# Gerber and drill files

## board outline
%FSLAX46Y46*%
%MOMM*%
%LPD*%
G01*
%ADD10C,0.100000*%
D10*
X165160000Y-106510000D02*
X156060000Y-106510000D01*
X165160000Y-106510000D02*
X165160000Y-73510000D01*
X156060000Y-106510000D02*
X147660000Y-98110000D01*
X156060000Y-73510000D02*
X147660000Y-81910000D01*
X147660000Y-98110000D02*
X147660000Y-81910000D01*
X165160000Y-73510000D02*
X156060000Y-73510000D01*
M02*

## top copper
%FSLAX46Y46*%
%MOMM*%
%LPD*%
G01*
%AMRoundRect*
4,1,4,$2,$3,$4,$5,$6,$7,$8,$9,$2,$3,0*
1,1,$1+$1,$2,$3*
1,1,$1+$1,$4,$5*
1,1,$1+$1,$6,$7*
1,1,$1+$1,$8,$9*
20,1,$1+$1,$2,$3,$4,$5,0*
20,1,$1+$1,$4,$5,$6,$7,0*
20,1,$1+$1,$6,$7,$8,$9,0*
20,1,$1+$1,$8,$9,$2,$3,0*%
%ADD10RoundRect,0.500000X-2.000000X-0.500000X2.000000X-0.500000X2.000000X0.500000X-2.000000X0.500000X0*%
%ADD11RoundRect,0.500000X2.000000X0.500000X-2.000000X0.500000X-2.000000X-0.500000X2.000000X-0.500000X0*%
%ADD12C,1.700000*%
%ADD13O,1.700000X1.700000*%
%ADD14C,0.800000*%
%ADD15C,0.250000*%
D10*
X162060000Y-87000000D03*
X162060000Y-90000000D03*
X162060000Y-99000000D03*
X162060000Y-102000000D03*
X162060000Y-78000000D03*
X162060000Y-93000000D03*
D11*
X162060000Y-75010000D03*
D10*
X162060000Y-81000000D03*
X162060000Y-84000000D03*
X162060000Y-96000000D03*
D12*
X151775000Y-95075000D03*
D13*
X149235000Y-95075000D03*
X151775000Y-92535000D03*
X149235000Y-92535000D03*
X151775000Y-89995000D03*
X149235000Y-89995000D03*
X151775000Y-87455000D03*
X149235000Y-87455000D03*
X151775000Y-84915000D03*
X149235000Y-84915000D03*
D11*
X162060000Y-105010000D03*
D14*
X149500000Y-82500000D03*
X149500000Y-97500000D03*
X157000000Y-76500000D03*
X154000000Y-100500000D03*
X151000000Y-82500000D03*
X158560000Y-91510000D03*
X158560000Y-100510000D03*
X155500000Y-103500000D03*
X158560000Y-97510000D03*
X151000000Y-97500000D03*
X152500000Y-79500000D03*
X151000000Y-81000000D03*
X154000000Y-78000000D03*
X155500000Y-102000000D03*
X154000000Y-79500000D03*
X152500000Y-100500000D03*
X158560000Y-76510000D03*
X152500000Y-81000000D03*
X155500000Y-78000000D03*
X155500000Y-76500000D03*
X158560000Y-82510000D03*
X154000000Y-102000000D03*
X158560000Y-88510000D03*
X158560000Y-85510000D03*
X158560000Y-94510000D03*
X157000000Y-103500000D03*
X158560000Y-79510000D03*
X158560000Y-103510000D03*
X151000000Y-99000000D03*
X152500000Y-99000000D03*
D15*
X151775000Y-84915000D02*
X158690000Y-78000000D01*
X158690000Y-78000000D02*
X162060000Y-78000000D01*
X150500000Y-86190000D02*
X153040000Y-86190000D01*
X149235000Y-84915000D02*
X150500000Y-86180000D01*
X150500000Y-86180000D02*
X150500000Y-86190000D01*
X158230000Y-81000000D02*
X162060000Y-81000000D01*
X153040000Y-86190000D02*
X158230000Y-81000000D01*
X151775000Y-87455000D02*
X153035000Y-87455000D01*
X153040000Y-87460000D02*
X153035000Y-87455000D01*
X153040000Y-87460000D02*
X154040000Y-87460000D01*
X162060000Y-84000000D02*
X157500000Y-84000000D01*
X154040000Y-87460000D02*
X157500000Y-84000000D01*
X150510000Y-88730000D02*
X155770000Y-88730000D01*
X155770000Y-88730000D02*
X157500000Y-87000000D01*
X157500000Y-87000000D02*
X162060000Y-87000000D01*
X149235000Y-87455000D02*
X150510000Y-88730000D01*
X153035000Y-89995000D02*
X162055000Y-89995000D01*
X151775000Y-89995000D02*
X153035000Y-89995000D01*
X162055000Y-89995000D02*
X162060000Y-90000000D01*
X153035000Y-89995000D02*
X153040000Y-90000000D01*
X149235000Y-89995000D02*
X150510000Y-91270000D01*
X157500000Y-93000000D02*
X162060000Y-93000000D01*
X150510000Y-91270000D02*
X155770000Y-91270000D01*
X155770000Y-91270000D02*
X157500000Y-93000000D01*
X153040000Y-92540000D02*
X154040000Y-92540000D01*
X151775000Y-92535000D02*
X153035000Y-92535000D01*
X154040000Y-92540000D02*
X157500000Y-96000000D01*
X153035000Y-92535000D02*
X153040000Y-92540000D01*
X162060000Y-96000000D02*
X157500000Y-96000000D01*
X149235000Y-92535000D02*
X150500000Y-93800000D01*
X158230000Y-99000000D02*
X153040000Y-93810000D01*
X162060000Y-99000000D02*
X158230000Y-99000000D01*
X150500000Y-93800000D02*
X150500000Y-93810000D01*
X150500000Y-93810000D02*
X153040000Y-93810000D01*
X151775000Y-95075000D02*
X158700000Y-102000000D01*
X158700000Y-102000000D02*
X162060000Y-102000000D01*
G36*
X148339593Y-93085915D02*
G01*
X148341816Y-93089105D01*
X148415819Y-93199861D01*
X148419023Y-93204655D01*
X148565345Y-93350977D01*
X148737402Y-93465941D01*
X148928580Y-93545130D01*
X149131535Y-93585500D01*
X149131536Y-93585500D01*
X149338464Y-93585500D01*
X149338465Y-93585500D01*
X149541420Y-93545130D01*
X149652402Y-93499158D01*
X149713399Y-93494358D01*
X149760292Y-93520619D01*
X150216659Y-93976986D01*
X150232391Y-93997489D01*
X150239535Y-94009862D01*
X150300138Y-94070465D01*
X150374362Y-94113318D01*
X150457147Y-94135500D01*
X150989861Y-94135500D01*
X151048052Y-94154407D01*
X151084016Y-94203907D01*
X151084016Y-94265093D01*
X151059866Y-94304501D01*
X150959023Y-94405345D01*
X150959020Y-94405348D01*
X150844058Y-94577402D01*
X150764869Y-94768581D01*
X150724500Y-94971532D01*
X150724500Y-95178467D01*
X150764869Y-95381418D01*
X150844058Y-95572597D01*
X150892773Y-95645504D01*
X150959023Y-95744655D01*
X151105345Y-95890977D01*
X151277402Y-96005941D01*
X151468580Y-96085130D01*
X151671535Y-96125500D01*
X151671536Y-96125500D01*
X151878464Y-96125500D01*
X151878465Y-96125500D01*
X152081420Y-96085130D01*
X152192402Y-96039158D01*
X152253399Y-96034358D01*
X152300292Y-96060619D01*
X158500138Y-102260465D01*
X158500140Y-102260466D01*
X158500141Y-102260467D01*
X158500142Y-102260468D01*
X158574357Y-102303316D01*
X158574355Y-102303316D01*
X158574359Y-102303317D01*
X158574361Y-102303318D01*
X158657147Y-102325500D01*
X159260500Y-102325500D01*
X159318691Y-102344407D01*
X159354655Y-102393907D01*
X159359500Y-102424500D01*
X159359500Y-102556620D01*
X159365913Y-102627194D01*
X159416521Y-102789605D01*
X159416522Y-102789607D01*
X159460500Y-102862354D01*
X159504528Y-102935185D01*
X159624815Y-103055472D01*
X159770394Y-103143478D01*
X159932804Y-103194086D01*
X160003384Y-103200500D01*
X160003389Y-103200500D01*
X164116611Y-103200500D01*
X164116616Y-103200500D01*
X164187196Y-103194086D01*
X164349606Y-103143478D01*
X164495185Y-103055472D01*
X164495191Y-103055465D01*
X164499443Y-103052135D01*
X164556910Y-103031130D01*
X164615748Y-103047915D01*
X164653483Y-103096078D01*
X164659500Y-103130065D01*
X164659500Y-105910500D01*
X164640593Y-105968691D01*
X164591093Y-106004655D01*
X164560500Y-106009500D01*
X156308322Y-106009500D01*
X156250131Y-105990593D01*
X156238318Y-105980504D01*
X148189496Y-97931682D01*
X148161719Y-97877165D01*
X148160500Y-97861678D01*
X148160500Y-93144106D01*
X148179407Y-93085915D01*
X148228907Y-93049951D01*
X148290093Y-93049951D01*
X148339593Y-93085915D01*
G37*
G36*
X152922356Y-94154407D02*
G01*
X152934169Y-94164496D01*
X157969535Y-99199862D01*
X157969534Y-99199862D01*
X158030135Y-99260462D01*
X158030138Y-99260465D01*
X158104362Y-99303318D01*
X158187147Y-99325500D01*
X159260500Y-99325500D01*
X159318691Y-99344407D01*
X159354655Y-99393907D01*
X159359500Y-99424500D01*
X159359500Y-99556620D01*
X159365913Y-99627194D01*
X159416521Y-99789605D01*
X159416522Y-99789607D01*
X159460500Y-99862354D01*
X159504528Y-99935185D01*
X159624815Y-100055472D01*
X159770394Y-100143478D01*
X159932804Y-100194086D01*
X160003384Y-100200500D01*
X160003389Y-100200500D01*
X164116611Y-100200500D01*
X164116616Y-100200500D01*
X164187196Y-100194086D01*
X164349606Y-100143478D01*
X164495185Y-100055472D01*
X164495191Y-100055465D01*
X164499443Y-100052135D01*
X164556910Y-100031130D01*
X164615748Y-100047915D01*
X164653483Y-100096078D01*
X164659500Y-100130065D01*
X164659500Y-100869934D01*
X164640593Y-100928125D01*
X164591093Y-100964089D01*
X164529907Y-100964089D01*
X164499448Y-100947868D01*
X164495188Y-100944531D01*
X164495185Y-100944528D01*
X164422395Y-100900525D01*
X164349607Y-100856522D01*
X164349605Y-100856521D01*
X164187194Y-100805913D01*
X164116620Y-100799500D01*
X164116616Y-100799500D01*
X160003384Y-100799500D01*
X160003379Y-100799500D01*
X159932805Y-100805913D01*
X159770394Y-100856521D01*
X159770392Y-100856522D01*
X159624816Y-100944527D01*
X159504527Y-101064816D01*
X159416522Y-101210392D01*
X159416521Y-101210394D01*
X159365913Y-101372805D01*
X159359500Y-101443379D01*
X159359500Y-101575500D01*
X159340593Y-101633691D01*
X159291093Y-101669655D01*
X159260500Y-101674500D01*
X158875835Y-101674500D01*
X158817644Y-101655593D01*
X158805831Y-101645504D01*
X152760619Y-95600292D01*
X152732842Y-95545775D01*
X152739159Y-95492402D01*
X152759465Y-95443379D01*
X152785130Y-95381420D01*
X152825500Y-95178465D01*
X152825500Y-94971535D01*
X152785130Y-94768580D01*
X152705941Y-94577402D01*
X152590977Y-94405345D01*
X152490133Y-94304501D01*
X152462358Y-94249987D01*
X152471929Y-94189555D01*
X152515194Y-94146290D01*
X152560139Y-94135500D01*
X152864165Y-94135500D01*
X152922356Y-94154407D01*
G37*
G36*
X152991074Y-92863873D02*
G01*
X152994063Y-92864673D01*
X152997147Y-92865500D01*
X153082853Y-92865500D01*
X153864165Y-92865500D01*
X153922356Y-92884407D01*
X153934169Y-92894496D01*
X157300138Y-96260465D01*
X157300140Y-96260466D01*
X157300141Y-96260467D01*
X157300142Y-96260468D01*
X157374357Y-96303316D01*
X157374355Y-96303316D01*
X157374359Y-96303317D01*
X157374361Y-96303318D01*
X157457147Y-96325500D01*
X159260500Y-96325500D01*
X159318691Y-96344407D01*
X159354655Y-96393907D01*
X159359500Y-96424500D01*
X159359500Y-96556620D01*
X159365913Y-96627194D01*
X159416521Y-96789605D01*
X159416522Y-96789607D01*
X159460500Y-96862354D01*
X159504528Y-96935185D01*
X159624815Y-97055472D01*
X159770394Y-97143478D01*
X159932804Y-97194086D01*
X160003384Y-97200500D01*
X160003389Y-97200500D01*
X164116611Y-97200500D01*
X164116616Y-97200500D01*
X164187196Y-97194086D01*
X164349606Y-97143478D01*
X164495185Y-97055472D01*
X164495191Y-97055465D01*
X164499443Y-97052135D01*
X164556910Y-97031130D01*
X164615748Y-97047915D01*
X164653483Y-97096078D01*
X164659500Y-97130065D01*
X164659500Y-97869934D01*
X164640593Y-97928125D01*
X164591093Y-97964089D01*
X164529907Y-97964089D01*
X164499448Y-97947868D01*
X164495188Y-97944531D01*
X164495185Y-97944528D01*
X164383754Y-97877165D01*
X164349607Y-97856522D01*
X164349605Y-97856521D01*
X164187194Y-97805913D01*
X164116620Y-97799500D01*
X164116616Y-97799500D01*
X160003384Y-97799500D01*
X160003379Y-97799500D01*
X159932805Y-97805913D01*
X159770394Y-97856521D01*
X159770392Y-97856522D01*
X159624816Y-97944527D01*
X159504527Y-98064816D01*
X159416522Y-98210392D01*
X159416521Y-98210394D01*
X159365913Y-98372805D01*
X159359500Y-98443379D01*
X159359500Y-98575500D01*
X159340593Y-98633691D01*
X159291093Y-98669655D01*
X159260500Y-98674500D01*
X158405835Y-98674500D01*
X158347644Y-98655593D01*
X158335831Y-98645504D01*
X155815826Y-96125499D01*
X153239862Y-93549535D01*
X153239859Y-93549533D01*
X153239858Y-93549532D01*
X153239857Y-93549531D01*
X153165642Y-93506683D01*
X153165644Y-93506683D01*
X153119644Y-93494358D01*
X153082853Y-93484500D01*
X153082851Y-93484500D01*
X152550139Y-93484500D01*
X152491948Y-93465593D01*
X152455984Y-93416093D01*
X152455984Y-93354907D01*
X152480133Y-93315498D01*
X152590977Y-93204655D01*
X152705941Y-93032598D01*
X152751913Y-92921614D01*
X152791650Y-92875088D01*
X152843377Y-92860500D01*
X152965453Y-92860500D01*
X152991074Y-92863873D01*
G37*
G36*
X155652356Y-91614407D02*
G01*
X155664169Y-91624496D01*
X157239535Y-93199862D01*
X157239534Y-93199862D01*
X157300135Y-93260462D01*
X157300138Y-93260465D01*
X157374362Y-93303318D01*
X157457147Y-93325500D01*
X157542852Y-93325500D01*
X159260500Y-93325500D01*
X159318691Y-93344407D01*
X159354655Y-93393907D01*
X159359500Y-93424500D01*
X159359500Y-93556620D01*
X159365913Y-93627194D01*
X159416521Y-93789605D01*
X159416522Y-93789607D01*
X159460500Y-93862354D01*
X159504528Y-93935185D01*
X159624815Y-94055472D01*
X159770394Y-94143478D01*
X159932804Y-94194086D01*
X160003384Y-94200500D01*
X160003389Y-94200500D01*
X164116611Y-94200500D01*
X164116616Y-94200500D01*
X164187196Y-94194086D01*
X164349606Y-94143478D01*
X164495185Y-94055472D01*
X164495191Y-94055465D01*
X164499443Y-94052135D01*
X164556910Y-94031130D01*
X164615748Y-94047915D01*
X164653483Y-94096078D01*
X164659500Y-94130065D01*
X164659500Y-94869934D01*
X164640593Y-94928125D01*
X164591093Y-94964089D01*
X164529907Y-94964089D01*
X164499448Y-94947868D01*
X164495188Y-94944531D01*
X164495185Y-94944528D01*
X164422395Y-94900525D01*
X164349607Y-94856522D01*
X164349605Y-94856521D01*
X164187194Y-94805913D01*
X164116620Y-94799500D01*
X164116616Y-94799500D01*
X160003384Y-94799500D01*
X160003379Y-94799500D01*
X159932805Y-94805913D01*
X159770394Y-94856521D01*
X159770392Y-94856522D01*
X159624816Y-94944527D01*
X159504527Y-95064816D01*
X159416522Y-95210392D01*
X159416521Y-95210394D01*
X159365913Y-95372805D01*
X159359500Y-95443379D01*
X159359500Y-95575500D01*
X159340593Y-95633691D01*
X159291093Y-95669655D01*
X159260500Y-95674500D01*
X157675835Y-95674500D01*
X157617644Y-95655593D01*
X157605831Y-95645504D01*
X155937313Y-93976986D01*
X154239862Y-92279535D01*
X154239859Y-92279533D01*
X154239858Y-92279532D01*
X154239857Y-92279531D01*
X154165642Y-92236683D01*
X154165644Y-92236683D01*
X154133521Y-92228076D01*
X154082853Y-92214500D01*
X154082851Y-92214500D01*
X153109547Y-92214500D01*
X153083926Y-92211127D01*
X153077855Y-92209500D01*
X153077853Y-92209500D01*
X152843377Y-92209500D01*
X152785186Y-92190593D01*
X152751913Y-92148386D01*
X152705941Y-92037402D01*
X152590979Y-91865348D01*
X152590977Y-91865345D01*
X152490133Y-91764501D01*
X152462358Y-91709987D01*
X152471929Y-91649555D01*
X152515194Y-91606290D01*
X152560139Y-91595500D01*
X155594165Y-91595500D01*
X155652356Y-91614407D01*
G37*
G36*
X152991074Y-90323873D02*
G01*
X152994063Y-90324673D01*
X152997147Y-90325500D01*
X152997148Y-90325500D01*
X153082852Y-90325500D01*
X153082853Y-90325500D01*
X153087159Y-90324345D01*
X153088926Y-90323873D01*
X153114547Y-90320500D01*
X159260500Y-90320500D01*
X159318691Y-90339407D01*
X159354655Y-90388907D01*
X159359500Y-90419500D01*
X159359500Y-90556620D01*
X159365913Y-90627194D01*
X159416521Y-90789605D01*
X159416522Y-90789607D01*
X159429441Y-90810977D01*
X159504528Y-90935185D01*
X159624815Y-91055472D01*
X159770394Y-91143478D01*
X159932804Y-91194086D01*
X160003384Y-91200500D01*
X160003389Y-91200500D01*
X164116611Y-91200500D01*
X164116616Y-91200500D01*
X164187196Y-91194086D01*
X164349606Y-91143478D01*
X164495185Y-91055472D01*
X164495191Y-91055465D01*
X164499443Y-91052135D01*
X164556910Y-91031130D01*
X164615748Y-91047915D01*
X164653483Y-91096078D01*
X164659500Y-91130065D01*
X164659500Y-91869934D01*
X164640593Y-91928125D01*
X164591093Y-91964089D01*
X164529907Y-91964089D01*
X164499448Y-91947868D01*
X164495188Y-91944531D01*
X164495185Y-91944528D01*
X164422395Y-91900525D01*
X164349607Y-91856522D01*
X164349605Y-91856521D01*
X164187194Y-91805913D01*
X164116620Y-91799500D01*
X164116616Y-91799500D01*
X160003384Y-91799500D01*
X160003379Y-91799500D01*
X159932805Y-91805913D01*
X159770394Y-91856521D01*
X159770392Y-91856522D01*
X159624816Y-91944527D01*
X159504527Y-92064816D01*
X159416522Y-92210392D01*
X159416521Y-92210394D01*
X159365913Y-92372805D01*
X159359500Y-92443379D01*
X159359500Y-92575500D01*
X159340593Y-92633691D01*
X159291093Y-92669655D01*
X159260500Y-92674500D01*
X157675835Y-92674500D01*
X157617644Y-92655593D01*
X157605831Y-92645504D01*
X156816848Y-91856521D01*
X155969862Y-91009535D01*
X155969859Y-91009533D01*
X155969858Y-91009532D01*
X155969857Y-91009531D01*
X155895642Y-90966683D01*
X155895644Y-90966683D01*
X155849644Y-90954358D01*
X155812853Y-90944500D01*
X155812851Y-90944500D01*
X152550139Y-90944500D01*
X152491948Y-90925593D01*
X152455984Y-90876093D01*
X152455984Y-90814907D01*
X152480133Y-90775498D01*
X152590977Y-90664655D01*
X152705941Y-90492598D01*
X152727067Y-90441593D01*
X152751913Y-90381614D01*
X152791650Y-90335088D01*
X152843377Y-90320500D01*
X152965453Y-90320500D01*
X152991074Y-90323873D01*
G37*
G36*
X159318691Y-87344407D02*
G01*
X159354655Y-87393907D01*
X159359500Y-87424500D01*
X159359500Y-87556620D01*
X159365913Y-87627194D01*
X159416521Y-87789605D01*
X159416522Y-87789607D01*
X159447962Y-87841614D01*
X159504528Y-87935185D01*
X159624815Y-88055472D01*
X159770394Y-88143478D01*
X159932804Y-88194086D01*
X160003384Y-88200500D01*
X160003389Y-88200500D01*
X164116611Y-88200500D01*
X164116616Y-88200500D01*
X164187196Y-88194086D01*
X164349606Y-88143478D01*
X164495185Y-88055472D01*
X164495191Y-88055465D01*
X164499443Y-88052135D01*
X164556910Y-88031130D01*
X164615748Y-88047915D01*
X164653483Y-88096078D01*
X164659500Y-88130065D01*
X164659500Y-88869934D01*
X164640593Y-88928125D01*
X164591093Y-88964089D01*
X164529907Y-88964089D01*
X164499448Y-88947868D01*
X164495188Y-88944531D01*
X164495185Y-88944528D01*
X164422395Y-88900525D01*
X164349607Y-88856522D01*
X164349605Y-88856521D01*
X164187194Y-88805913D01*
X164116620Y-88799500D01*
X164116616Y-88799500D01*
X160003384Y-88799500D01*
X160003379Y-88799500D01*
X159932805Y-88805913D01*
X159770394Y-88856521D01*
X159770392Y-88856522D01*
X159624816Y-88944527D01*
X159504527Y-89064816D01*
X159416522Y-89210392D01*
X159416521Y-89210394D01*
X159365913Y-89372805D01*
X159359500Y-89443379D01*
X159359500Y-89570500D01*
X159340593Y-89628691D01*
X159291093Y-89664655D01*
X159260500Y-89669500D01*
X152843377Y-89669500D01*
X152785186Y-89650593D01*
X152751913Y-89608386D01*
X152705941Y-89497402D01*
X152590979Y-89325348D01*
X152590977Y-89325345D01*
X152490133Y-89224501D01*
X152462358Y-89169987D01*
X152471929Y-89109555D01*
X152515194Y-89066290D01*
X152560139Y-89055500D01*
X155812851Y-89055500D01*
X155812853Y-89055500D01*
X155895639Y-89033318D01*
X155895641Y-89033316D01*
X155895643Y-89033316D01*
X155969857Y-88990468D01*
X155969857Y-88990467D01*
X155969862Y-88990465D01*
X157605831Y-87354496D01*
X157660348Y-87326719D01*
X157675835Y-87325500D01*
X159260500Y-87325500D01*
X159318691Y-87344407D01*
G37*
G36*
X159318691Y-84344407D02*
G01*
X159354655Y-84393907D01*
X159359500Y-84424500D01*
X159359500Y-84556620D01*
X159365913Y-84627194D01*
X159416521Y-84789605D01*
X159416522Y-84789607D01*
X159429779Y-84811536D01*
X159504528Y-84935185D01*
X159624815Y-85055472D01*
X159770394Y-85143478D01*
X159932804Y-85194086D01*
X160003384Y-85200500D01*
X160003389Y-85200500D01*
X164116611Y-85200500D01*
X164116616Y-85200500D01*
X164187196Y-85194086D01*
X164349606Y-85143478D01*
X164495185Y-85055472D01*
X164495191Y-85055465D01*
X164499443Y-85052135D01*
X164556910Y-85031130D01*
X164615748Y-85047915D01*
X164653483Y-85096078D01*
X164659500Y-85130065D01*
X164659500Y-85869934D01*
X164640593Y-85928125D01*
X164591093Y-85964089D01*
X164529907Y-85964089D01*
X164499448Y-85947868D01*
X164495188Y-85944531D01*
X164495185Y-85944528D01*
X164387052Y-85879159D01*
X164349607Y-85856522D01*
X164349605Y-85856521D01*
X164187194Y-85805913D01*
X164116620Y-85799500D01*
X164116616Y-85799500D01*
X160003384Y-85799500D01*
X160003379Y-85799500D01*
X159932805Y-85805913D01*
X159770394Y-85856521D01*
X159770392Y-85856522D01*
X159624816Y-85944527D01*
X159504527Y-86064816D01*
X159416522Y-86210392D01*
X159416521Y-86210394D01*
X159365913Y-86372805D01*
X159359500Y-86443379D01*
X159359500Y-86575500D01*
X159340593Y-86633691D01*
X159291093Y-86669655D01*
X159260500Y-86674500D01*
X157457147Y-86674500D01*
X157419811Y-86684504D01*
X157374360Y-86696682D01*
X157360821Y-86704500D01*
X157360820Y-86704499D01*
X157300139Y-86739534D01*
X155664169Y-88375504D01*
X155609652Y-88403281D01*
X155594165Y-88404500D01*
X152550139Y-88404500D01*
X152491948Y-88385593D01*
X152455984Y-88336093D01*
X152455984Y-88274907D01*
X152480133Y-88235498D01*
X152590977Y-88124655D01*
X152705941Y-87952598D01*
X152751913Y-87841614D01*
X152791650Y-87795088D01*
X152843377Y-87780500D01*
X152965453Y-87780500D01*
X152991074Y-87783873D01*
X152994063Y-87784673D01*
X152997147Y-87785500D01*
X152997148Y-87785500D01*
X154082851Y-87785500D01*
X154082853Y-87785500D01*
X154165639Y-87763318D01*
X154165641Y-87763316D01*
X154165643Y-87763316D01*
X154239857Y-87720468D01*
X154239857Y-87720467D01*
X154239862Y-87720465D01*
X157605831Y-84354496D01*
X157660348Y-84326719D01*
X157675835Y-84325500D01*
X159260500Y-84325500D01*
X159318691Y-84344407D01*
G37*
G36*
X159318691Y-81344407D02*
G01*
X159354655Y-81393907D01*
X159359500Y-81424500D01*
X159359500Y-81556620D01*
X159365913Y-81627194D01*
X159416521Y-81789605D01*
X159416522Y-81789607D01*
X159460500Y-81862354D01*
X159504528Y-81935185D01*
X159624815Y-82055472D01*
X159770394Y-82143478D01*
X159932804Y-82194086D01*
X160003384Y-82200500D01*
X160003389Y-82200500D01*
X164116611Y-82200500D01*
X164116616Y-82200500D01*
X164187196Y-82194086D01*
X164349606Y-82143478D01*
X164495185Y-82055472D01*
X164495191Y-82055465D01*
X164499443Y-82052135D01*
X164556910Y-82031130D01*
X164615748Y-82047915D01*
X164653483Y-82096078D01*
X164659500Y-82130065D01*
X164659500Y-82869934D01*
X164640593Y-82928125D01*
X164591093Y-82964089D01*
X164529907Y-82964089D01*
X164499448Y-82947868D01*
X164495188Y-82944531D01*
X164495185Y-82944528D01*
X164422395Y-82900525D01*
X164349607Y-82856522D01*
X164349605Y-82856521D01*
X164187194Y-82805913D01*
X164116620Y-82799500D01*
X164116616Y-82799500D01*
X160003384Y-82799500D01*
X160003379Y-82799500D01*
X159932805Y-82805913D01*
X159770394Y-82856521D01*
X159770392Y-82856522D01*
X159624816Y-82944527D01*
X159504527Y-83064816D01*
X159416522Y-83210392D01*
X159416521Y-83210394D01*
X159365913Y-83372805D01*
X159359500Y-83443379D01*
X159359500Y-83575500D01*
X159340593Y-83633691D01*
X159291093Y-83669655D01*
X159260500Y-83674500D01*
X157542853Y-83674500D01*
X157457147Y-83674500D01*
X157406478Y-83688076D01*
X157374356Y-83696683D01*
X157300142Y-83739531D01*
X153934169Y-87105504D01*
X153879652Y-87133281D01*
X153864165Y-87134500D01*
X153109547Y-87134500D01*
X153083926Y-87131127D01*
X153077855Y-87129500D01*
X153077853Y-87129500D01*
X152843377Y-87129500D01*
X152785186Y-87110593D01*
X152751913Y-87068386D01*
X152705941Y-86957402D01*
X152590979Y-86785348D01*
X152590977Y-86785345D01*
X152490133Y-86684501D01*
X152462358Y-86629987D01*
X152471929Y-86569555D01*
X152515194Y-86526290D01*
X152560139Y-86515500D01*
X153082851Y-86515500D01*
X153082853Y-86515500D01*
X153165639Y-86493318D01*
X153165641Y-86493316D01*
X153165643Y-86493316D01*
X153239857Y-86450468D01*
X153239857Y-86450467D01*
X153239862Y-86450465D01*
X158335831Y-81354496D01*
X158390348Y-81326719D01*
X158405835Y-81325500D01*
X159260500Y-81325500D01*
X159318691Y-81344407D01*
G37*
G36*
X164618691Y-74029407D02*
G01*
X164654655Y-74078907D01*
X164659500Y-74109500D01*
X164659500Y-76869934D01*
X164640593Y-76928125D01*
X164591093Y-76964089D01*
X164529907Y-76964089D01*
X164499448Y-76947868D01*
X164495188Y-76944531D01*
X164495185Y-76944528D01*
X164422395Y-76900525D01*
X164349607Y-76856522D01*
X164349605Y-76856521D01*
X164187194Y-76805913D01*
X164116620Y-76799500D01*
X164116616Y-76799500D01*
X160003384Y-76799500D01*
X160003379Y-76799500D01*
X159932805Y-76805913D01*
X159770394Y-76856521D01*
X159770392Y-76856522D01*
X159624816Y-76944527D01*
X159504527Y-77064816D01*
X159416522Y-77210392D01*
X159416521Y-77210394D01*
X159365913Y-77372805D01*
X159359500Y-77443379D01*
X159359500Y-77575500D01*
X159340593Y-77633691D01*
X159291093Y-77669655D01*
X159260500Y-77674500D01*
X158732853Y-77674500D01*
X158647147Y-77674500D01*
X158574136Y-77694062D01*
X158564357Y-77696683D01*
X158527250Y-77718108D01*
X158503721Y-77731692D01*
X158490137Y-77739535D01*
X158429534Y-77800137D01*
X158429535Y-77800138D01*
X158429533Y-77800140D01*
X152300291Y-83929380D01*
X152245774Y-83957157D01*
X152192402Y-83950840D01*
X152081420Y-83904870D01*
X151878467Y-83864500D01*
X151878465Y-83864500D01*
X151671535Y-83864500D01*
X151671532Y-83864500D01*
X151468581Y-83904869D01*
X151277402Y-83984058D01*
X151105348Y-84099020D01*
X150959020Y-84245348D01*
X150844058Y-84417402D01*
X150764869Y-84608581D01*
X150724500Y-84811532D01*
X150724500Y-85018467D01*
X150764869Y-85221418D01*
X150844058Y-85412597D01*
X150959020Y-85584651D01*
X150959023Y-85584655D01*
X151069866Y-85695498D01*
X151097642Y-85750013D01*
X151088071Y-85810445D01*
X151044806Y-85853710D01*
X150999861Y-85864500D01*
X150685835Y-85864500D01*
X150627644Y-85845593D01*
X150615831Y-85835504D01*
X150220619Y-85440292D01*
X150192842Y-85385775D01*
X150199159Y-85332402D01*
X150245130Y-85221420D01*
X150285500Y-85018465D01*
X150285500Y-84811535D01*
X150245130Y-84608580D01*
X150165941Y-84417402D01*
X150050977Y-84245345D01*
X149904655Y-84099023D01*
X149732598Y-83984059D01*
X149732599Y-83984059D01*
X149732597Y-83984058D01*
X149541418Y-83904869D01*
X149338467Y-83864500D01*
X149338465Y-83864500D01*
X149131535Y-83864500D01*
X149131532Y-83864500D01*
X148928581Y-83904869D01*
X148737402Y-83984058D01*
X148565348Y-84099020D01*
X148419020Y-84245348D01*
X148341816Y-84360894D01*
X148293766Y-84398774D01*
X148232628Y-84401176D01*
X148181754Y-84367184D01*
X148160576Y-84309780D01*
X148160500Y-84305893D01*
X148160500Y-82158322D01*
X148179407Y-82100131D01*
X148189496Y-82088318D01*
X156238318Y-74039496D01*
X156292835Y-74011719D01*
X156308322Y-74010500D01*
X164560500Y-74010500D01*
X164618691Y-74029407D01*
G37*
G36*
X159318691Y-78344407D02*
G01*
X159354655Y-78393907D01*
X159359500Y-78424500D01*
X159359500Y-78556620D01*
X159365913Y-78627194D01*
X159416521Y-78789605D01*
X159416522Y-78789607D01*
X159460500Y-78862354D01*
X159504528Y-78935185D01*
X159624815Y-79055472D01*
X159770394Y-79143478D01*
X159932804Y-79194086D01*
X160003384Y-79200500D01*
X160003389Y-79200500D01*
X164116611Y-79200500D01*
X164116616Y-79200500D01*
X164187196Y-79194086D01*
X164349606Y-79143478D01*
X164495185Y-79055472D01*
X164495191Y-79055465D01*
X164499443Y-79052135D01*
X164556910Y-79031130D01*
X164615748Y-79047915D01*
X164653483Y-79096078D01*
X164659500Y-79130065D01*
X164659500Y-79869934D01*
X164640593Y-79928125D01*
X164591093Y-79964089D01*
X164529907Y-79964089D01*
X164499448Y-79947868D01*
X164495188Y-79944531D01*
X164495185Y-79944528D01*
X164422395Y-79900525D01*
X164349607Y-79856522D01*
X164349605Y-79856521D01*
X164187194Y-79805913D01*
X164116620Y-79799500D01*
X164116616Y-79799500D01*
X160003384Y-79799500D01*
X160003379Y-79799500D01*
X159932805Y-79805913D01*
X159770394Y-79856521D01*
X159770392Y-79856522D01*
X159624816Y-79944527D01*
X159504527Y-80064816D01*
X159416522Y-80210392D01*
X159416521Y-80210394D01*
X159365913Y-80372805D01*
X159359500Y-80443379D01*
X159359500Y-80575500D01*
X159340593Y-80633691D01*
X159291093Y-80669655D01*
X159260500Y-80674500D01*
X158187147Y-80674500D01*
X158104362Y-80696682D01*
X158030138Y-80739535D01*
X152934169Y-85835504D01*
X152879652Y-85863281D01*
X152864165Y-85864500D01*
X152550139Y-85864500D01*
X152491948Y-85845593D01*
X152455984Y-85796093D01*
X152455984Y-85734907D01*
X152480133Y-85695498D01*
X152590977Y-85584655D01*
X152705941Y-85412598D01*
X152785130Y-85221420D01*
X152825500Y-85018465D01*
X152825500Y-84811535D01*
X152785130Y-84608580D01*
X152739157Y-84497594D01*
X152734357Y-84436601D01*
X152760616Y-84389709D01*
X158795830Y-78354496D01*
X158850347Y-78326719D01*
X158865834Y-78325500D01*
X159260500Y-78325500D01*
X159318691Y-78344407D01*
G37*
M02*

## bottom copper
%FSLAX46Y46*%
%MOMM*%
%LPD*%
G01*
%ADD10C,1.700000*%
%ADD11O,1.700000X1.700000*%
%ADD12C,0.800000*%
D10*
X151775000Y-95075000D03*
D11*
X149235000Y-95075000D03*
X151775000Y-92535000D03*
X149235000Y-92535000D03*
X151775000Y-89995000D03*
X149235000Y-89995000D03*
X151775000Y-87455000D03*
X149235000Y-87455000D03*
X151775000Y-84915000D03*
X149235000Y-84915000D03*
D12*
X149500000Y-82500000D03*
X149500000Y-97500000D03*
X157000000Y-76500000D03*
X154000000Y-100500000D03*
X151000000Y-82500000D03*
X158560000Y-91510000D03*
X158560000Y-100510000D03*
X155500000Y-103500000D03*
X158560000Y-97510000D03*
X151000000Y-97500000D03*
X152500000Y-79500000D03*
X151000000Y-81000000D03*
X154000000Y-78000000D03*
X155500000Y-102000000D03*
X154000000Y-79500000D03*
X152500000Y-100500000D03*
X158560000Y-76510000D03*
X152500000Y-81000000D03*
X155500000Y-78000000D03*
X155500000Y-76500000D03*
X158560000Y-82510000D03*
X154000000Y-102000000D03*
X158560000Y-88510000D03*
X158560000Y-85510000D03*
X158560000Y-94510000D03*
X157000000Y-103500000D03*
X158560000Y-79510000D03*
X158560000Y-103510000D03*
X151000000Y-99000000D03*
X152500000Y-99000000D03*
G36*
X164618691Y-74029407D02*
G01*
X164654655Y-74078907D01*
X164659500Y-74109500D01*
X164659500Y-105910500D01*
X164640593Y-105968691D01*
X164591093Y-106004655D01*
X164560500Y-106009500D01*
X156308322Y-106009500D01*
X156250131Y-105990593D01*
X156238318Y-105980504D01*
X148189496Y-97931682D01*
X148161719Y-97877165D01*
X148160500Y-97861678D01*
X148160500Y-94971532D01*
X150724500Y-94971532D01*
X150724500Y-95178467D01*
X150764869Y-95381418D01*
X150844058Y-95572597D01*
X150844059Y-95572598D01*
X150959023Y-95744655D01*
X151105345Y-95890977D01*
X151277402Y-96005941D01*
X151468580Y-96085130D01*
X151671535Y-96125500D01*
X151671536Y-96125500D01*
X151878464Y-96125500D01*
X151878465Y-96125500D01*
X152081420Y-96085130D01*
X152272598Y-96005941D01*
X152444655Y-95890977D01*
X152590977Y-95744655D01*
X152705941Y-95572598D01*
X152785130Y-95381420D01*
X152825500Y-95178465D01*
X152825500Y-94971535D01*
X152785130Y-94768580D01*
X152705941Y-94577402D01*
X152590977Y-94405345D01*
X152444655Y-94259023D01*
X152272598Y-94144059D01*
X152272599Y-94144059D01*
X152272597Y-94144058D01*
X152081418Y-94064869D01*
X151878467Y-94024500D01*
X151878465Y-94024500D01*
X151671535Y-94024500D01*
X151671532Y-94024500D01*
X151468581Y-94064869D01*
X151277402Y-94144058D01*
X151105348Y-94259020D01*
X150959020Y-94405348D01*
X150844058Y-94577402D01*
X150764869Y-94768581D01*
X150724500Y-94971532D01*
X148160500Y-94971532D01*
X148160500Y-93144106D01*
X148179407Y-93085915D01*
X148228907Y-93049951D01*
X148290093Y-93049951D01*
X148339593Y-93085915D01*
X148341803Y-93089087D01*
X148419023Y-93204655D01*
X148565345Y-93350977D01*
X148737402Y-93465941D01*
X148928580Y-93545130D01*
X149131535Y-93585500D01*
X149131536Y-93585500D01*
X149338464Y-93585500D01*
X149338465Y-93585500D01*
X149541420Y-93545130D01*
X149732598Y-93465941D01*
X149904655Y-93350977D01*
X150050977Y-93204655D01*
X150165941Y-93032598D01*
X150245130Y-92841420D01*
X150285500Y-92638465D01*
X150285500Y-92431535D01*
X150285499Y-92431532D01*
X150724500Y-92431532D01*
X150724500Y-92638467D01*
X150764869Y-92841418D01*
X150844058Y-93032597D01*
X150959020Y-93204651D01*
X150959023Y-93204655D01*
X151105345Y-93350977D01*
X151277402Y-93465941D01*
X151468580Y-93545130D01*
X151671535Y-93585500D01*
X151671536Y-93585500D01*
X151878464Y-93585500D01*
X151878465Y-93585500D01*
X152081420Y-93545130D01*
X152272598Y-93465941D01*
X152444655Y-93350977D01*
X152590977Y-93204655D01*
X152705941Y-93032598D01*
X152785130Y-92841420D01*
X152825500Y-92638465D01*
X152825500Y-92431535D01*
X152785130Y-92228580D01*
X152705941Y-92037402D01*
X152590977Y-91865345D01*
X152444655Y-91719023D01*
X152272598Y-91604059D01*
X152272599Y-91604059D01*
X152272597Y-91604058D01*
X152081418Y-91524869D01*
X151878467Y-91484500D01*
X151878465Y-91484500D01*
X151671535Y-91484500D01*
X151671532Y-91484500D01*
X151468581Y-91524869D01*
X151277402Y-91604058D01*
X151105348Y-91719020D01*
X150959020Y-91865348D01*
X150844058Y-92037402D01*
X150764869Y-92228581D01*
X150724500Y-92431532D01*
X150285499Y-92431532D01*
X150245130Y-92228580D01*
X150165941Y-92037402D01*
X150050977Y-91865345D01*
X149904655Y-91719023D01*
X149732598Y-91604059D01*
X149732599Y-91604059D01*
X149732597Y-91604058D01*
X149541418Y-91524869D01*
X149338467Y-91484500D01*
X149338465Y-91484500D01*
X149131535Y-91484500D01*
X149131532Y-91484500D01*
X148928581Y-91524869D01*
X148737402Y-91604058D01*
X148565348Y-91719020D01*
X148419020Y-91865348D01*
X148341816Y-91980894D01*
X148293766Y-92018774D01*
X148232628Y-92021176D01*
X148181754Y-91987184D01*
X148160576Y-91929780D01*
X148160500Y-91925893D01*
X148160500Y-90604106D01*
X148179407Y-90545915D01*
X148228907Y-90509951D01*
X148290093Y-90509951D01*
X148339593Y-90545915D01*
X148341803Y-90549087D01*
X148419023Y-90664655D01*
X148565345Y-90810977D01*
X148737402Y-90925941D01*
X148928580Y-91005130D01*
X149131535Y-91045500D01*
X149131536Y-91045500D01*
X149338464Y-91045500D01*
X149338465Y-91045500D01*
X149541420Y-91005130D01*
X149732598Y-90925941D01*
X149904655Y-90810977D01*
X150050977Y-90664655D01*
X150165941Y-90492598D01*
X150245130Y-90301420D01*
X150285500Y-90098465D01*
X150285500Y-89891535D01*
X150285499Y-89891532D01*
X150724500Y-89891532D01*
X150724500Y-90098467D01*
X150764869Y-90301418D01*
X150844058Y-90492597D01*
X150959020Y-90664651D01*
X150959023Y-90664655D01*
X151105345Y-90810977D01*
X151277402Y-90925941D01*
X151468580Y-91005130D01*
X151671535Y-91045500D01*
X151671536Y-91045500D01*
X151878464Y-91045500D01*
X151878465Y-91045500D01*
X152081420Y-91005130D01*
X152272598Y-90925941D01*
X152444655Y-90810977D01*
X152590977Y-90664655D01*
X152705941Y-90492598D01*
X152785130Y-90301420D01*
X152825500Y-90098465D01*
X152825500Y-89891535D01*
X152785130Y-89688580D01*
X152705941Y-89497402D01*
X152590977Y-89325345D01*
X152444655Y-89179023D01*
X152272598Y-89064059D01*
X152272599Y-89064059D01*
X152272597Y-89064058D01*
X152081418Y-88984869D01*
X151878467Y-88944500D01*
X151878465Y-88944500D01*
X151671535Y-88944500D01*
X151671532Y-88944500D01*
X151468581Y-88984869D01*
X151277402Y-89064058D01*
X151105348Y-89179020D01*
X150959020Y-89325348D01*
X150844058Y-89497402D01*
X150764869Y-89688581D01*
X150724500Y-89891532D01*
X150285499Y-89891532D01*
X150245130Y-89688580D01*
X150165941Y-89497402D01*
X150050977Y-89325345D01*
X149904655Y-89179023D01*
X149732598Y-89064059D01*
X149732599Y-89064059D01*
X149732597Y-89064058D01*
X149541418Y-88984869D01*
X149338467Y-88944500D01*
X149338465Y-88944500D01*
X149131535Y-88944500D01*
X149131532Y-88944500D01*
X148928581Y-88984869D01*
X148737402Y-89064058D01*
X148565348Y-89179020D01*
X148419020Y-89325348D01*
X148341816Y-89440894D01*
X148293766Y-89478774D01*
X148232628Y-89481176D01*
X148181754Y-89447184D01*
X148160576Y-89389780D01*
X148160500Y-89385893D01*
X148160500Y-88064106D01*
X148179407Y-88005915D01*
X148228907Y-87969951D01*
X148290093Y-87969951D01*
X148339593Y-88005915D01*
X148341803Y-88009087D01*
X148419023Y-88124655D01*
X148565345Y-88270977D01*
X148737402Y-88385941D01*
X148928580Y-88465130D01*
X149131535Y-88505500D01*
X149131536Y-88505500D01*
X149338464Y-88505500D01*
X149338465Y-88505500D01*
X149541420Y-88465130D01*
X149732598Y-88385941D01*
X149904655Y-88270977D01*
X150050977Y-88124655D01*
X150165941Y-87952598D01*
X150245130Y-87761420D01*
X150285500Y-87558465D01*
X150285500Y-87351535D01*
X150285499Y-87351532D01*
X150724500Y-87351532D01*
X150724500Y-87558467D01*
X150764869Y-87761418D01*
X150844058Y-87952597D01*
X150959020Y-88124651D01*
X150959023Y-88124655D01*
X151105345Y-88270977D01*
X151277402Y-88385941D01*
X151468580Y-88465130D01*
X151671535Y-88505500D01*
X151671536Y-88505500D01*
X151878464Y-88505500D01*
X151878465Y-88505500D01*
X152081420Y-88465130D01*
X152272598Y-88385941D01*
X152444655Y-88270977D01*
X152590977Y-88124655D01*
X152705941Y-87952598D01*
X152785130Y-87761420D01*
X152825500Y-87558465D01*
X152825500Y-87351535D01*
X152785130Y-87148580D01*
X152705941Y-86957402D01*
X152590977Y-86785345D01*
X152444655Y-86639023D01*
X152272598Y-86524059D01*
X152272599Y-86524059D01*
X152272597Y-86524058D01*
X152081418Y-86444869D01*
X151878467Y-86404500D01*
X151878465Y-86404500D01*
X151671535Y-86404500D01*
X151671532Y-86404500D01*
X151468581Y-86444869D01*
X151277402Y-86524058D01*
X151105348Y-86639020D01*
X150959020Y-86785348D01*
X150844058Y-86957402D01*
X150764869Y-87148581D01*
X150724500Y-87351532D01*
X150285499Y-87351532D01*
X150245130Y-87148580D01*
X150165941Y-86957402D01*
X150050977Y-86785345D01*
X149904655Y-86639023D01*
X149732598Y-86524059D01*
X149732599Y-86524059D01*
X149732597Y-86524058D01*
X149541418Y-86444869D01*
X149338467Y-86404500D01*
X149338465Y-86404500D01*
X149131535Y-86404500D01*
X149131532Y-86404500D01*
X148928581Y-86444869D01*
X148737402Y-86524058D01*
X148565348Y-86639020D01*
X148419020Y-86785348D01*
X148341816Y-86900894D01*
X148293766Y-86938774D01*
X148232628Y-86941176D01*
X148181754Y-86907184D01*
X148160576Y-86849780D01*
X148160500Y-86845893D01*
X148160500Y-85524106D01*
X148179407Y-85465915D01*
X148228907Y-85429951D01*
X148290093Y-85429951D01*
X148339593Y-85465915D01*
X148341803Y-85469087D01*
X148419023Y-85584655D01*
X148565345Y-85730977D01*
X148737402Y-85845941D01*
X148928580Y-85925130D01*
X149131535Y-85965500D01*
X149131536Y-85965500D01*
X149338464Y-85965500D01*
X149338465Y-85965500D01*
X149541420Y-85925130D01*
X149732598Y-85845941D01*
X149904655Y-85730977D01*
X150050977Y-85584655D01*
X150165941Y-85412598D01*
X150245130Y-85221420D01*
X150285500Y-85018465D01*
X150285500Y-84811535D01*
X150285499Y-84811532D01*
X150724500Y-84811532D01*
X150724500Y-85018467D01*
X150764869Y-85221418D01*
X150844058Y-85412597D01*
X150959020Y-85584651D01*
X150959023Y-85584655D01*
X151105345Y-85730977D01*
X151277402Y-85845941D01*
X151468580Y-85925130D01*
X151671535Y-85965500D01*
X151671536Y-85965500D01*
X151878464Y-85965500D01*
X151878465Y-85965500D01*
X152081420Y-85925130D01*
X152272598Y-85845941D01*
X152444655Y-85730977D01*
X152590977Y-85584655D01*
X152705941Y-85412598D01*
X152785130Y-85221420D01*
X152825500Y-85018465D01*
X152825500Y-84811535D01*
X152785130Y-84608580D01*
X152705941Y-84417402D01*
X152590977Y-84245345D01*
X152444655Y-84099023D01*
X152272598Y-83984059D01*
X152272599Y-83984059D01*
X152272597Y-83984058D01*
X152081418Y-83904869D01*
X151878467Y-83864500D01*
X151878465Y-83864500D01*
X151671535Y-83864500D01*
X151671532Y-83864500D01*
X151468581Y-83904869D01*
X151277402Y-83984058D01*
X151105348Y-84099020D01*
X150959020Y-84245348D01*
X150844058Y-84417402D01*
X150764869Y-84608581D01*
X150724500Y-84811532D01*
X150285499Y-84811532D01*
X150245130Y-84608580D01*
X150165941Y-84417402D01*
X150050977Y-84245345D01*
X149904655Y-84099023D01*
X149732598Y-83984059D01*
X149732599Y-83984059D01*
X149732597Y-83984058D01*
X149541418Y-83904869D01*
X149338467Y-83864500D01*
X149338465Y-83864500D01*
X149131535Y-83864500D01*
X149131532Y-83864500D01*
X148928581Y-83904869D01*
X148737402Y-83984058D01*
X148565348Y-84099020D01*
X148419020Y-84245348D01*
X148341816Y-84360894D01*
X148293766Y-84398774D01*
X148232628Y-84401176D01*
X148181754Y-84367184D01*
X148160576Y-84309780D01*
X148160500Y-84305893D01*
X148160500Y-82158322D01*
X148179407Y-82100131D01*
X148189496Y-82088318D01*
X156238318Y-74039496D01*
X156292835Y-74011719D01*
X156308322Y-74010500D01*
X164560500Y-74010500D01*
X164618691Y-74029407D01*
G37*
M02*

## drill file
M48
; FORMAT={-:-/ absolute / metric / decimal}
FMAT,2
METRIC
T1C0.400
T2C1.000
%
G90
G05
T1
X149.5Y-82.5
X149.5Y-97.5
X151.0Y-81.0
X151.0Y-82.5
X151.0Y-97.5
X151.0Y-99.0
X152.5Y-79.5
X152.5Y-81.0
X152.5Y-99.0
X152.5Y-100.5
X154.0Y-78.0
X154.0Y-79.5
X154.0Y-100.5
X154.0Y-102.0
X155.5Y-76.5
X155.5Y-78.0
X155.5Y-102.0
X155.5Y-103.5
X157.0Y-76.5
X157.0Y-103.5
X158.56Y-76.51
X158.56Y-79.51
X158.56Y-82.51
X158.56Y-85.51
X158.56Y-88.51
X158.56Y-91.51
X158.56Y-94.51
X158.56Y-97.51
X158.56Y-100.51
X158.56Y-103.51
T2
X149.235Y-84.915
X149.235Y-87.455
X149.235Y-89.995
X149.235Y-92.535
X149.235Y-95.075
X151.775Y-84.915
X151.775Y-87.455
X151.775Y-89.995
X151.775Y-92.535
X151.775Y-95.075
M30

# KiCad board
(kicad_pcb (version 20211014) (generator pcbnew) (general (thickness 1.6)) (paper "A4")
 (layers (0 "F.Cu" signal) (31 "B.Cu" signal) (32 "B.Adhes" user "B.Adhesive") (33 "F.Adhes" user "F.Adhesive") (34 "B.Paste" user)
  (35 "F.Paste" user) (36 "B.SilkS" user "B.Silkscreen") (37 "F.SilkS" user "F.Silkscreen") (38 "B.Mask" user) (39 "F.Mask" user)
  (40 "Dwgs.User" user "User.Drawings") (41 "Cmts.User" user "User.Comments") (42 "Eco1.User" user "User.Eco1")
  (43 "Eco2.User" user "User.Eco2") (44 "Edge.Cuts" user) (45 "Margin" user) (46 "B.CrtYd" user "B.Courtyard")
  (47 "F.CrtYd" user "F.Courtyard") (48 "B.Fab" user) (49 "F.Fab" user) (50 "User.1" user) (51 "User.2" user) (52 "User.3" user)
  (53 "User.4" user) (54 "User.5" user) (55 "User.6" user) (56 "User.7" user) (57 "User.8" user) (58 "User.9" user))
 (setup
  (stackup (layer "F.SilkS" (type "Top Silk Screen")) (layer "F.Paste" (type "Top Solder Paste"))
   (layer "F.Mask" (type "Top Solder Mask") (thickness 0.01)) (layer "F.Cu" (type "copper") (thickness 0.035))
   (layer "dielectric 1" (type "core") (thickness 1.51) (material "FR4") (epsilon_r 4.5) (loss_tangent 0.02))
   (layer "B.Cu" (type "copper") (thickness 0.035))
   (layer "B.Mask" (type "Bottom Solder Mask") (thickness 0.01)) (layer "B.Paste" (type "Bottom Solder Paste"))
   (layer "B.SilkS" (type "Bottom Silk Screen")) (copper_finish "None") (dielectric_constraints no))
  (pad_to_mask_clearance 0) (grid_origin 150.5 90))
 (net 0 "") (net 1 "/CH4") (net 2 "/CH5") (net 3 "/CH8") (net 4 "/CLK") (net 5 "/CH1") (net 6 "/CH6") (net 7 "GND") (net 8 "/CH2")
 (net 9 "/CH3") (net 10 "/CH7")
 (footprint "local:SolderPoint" (layer "F.Cu") (at 162.06 87)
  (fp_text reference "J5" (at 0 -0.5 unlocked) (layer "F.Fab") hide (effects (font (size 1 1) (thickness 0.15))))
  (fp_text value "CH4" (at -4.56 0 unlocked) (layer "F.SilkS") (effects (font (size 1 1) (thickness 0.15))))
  (pad "1" smd roundrect (at 0 0) (size 5 2) (layers "F.Cu" "F.Paste" "F.Mask") (roundrect_rratio 0.25) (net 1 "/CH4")))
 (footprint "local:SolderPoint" (layer "F.Cu") (at 162.06 90)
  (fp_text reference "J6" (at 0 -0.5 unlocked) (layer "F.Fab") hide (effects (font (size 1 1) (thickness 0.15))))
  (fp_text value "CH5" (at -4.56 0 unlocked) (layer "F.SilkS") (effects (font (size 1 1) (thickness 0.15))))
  (pad "1" smd roundrect (at 0 0) (size 5 2) (layers "F.Cu" "F.Paste" "F.Mask") (roundrect_rratio 0.25) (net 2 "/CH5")))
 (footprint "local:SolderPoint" (layer "F.Cu") (at 162.06 99)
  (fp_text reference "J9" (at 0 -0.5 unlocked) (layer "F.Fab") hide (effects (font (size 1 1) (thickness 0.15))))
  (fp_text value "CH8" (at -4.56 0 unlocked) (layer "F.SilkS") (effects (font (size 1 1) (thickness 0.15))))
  (pad "1" smd roundrect (at 0 0) (size 5 2) (layers "F.Cu" "F.Paste" "F.Mask") (roundrect_rratio 0.25) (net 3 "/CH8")))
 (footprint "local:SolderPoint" (layer "F.Cu") (at 162.06 102)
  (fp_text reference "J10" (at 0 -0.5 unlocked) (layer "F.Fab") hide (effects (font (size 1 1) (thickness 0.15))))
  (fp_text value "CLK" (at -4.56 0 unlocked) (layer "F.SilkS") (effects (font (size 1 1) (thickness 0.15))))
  (pad "1" smd roundrect (at 0 0) (size 5 2) (layers "F.Cu" "F.Paste" "F.Mask") (roundrect_rratio 0.25) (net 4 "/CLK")))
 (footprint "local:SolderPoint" (layer "F.Cu") (at 162.06 78)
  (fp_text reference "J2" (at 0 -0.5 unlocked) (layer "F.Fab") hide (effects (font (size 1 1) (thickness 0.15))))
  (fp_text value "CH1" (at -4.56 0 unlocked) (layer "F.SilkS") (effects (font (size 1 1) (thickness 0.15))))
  (pad "1" smd roundrect (at 0 0) (size 5 2) (layers "F.Cu" "F.Paste" "F.Mask") (roundrect_rratio 0.25) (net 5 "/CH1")))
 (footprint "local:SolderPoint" (layer "F.Cu") (at 162.06 93)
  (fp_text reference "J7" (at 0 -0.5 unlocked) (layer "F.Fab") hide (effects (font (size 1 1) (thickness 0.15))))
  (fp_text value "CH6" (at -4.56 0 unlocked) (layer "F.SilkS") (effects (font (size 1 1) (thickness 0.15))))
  (pad "1" smd roundrect (at 0 0) (size 5 2) (layers "F.Cu" "F.Paste" "F.Mask") (roundrect_rratio 0.25) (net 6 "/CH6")))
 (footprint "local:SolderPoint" (layer "F.Cu") (at 162.06 75.01 180)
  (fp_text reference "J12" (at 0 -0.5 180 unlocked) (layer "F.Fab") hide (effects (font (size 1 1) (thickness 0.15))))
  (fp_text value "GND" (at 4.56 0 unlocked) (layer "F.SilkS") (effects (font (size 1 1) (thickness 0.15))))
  (pad "1" smd roundrect (at 0 0 180) (size 5 2) (layers "F.Cu" "F.Paste" "F.Mask") (roundrect_rratio 0.25) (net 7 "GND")))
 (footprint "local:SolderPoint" (layer "F.Cu") (at 162.06 81)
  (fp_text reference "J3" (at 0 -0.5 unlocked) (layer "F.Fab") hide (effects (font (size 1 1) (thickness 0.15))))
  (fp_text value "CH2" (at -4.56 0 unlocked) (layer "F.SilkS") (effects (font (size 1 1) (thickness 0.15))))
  (pad "1" smd roundrect (at 0 0) (size 5 2) (layers "F.Cu" "F.Paste" "F.Mask") (roundrect_rratio 0.25) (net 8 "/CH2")))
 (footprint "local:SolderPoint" (layer "F.Cu") (at 162.06 84)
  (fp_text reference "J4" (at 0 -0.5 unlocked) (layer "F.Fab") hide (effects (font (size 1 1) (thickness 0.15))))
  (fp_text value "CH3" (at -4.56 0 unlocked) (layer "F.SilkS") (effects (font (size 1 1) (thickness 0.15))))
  (pad "1" smd roundrect (at 0 0) (size 5 2) (layers "F.Cu" "F.Paste" "F.Mask") (roundrect_rratio 0.25) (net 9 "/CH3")))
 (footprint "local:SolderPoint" (layer "F.Cu") (at 162.06 96)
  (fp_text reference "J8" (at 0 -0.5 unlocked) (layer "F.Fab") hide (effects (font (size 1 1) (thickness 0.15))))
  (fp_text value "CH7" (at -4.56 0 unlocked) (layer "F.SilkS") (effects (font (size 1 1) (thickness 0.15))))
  (pad "1" smd roundrect (at 0 0) (size 5 2) (layers "F.Cu" "F.Paste" "F.Mask") (roundrect_rratio 0.25) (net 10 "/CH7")))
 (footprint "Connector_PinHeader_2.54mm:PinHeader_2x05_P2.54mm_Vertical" (layer "F.Cu") (at 151.775 95.075 180)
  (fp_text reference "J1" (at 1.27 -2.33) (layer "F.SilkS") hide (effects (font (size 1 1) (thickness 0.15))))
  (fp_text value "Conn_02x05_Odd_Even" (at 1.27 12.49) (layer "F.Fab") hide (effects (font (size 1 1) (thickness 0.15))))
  (pad "1" thru_hole circle (at 0 0 180) (size 1.7 1.7) (drill 1) (layers *.Cu *.Mask) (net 4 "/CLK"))
  (pad "2" thru_hole oval (at 2.54 0 180) (size 1.7 1.7) (drill 1) (layers *.Cu *.Mask) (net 7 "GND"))
  (pad "3" thru_hole oval (at 0 2.54 180) (size 1.7 1.7) (drill 1) (layers *.Cu *.Mask) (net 10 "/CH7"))
  (pad "4" thru_hole oval (at 2.54 2.54 180) (size 1.7 1.7) (drill 1) (layers *.Cu *.Mask) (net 3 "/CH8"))
  (pad "5" thru_hole oval (at 0 5.08 180) (size 1.7 1.7) (drill 1) (layers *.Cu *.Mask) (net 2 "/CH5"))
  (pad "6" thru_hole oval (at 2.54 5.08 180) (size 1.7 1.7) (drill 1) (layers *.Cu *.Mask) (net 6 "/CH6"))
  (pad "7" thru_hole oval (at 0 7.62 180) (size 1.7 1.7) (drill 1) (layers *.Cu *.Mask) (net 9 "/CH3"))
  (pad "8" thru_hole oval (at 2.54 7.62 180) (size 1.7 1.7) (drill 1) (layers *.Cu *.Mask) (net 1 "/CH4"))
  (pad "9" thru_hole oval (at 0 10.16 180) (size 1.7 1.7) (drill 1) (layers *.Cu *.Mask) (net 5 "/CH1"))
  (pad "10" thru_hole oval (at 2.54 10.16 180) (size 1.7 1.7) (drill 1) (layers *.Cu *.Mask) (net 8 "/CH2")))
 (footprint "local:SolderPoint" (layer "F.Cu") (at 162.06 105.01 180)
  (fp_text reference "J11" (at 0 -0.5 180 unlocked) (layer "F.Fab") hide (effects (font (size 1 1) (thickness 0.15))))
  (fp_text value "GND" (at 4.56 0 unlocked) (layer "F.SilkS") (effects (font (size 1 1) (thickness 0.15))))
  (pad "1" smd roundrect (at 0 0 180) (size 5 2) (layers "F.Cu" "F.Paste" "F.Mask") (roundrect_rratio 0.25) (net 7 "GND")))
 (gr_line (start 165.16 106.51) (end 156.06 106.51) (layer "Edge.Cuts") (width 0.1))
 (gr_line (start 165.16 106.51) (end 165.16 73.51) (layer "Edge.Cuts") (width 0.1))
 (gr_line (start 156.06 106.51) (end 147.66 98.11) (layer "Edge.Cuts") (width 0.1))
 (gr_line (start 156.06 73.51) (end 147.66 81.91) (layer "Edge.Cuts") (width 0.1))
 (gr_line (start 147.66 98.11) (end 147.66 81.91) (layer "Edge.Cuts") (width 0.1))
 (gr_line (start 165.16 73.51) (end 156.06 73.51) (layer "Edge.Cuts") (width 0.1))
 (segment (start 151.775 84.915) (end 158.69 78) (width 0.25) (layer "F.Cu") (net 5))
 (segment (start 158.69 78) (end 162.06 78) (width 0.25) (layer "F.Cu") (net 5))
 (segment (start 150.5 86.19) (end 153.04 86.19) (width 0.25) (layer "F.Cu") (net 8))
 (segment (start 149.235 84.915) (end 150.5 86.18) (width 0.25) (layer "F.Cu") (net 8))
 (segment (start 150.5 86.18) (end 150.5 86.19) (width 0.25) (layer "F.Cu") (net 8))
 (segment (start 158.23 81) (end 162.06 81) (width 0.25) (layer "F.Cu") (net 8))
 (segment (start 153.04 86.19) (end 158.23 81) (width 0.25) (layer "F.Cu") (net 8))
 (segment (start 151.775 87.455) (end 153.035 87.455) (width 0.25) (layer "F.Cu") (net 9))
 (segment (start 153.04 87.46) (end 153.035 87.455) (width 0.25) (layer "F.Cu") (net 9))
 (segment (start 153.04 87.46) (end 154.04 87.46) (width 0.25) (layer "F.Cu") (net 9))
 (segment (start 162.06 84) (end 157.5 84) (width 0.25) (layer "F.Cu") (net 9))
 (segment (start 154.04 87.46) (end 157.5 84) (width 0.25) (layer "F.Cu") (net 9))
 (segment (start 150.51 88.73) (end 155.77 88.73) (width 0.25) (layer "F.Cu") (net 1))
 (segment (start 155.77 88.73) (end 157.5 87) (width 0.25) (layer "F.Cu") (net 1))
 (segment (start 157.5 87) (end 162.06 87) (width 0.25) (layer "F.Cu") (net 1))
 (segment (start 149.235 87.455) (end 150.51 88.73) (width 0.25) (layer "F.Cu") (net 1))
 (segment (start 153.035 89.995) (end 162.055 89.995) (width 0.25) (layer "F.Cu") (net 2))
 (segment (start 151.775 89.995) (end 153.035 89.995) (width 0.25) (layer "F.Cu") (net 2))
 (segment (start 162.055 89.995) (end 162.06 90) (width 0.25) (layer "F.Cu") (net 2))
 (segment (start 153.035 89.995) (end 153.04 90) (width 0.25) (layer "F.Cu") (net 2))
 (segment (start 149.235 89.995) (end 150.51 91.27) (width 0.25) (layer "F.Cu") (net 6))
 (segment (start 157.5 93) (end 162.06 93) (width 0.25) (layer "F.Cu") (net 6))
 (segment (start 150.51 91.27) (end 155.77 91.27) (width 0.25) (layer "F.Cu") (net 6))
 (segment (start 155.77 91.27) (end 157.5 93) (width 0.25) (layer "F.Cu") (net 6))
 (segment (start 153.04 92.54) (end 154.04 92.54) (width 0.25) (layer "F.Cu") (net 10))
 (segment (start 151.775 92.535) (end 153.035 92.535) (width 0.25) (layer "F.Cu") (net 10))
 (segment (start 154.04 92.54) (end 157.5 96) (width 0.25) (layer "F.Cu") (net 10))
 (segment (start 153.035 92.535) (end 153.04 92.54) (width 0.25) (layer "F.Cu") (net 10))
 (segment (start 162.06 96) (end 157.5 96) (width 0.25) (layer "F.Cu") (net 10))
 (segment (start 149.235 92.535) (end 150.5 93.8) (width 0.25) (layer "F.Cu") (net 3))
 (segment (start 158.23 99) (end 153.04 93.81) (width 0.25) (layer "F.Cu") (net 3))
 (segment (start 162.06 99) (end 158.23 99) (width 0.25) (layer "F.Cu") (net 3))
 (segment (start 150.5 93.8) (end 150.5 93.81) (width 0.25) (layer "F.Cu") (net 3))
 (segment (start 150.5 93.81) (end 153.04 93.81) (width 0.25) (layer "F.Cu") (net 3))
 (segment (start 151.775 95.075) (end 158.7 102) (width 0.25) (layer "F.Cu") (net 4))
 (segment (start 158.7 102) (end 162.06 102) (width 0.25) (layer "F.Cu") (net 4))
 (via (at 149.5 82.5) (size 0.8) (drill 0.4) (layers "F.Cu" "B.Cu") (free) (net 7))
 (via (at 149.5 97.5) (size 0.8) (drill 0.4) (layers "F.Cu" "B.Cu") (free) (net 7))
 (via (at 157 76.5) (size 0.8) (drill 0.4) (layers "F.Cu" "B.Cu") (free) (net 7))
 (via (at 154 100.5) (size 0.8) (drill 0.4) (layers "F.Cu" "B.Cu") (free) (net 7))
 (via (at 151 82.5) (size 0.8) (drill 0.4) (layers "F.Cu" "B.Cu") (free) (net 7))
 (via (at 158.56 91.51) (size 0.8) (drill 0.4) (layers "F.Cu" "B.Cu") (free) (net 7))
 (via (at 158.56 100.51) (size 0.8) (drill 0.4) (layers "F.Cu" "B.Cu") (free) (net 7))
 (via (at 155.5 103.5) (size 0.8) (drill 0.4) (layers "F.Cu" "B.Cu") (free) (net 7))
 (via (at 158.56 97.51) (size 0.8) (drill 0.4) (layers "F.Cu" "B.Cu") (free) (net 7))
 (via (at 151 97.5) (size 0.8) (drill 0.4) (layers "F.Cu" "B.Cu") (free) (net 7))
 (via (at 152.5 79.5) (size 0.8) (drill 0.4) (layers "F.Cu" "B.Cu") (free) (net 7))
 (via (at 151 81) (size 0.8) (drill 0.4) (layers "F.Cu" "B.Cu") (free) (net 7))
 (via (at 154 78) (size 0.8) (drill 0.4) (layers "F.Cu" "B.Cu") (free) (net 7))
 (via (at 155.5 102) (size 0.8) (drill 0.4) (layers "F.Cu" "B.Cu") (free) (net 7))
 (via (at 154 79.5) (size 0.8) (drill 0.4) (layers "F.Cu" "B.Cu") (free) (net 7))
 (via (at 152.5 100.5) (size 0.8) (drill 0.4) (layers "F.Cu" "B.Cu") (free) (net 7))
 (via (at 158.56 76.51) (size 0.8) (drill 0.4) (layers "F.Cu" "B.Cu") (free) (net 7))
 (via (at 152.5 81) (size 0.8) (drill 0.4) (layers "F.Cu" "B.Cu") (free) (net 7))
 (via (at 155.5 78) (size 0.8) (drill 0.4) (layers "F.Cu" "B.Cu") (free) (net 7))
 (via (at 155.5 76.5) (size 0.8) (drill 0.4) (layers "F.Cu" "B.Cu") (free) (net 7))
 (via (at 158.56 82.51) (size 0.8) (drill 0.4) (layers "F.Cu" "B.Cu") (free) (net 7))
 (via (at 154 102) (size 0.8) (drill 0.4) (layers "F.Cu" "B.Cu") (free) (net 7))
 (via (at 158.56 88.51) (size 0.8) (drill 0.4) (layers "F.Cu" "B.Cu") (free) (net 7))
 (via (at 158.56 85.51) (size 0.8) (drill 0.4) (layers "F.Cu" "B.Cu") (free) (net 7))
 (via (at 158.56 94.51) (size 0.8) (drill 0.4) (layers "F.Cu" "B.Cu") (free) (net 7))
 (via (at 157 103.5) (size 0.8) (drill 0.4) (layers "F.Cu" "B.Cu") (free) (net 7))
 (via (at 158.56 79.51) (size 0.8) (drill 0.4) (layers "F.Cu" "B.Cu") (free) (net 7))
 (via (at 158.56 103.51) (size 0.8) (drill 0.4) (layers "F.Cu" "B.Cu") (free) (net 7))
 (via (at 151 99) (size 0.8) (drill 0.4) (layers "F.Cu" "B.Cu") (free) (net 7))
 (via (at 152.5 99) (size 0.8) (drill 0.4) (layers "F.Cu" "B.Cu") (free) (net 7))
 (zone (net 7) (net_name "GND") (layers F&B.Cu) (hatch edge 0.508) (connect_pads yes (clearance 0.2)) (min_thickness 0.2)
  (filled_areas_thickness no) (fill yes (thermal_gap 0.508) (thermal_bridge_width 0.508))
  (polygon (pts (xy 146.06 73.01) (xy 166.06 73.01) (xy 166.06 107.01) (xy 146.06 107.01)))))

